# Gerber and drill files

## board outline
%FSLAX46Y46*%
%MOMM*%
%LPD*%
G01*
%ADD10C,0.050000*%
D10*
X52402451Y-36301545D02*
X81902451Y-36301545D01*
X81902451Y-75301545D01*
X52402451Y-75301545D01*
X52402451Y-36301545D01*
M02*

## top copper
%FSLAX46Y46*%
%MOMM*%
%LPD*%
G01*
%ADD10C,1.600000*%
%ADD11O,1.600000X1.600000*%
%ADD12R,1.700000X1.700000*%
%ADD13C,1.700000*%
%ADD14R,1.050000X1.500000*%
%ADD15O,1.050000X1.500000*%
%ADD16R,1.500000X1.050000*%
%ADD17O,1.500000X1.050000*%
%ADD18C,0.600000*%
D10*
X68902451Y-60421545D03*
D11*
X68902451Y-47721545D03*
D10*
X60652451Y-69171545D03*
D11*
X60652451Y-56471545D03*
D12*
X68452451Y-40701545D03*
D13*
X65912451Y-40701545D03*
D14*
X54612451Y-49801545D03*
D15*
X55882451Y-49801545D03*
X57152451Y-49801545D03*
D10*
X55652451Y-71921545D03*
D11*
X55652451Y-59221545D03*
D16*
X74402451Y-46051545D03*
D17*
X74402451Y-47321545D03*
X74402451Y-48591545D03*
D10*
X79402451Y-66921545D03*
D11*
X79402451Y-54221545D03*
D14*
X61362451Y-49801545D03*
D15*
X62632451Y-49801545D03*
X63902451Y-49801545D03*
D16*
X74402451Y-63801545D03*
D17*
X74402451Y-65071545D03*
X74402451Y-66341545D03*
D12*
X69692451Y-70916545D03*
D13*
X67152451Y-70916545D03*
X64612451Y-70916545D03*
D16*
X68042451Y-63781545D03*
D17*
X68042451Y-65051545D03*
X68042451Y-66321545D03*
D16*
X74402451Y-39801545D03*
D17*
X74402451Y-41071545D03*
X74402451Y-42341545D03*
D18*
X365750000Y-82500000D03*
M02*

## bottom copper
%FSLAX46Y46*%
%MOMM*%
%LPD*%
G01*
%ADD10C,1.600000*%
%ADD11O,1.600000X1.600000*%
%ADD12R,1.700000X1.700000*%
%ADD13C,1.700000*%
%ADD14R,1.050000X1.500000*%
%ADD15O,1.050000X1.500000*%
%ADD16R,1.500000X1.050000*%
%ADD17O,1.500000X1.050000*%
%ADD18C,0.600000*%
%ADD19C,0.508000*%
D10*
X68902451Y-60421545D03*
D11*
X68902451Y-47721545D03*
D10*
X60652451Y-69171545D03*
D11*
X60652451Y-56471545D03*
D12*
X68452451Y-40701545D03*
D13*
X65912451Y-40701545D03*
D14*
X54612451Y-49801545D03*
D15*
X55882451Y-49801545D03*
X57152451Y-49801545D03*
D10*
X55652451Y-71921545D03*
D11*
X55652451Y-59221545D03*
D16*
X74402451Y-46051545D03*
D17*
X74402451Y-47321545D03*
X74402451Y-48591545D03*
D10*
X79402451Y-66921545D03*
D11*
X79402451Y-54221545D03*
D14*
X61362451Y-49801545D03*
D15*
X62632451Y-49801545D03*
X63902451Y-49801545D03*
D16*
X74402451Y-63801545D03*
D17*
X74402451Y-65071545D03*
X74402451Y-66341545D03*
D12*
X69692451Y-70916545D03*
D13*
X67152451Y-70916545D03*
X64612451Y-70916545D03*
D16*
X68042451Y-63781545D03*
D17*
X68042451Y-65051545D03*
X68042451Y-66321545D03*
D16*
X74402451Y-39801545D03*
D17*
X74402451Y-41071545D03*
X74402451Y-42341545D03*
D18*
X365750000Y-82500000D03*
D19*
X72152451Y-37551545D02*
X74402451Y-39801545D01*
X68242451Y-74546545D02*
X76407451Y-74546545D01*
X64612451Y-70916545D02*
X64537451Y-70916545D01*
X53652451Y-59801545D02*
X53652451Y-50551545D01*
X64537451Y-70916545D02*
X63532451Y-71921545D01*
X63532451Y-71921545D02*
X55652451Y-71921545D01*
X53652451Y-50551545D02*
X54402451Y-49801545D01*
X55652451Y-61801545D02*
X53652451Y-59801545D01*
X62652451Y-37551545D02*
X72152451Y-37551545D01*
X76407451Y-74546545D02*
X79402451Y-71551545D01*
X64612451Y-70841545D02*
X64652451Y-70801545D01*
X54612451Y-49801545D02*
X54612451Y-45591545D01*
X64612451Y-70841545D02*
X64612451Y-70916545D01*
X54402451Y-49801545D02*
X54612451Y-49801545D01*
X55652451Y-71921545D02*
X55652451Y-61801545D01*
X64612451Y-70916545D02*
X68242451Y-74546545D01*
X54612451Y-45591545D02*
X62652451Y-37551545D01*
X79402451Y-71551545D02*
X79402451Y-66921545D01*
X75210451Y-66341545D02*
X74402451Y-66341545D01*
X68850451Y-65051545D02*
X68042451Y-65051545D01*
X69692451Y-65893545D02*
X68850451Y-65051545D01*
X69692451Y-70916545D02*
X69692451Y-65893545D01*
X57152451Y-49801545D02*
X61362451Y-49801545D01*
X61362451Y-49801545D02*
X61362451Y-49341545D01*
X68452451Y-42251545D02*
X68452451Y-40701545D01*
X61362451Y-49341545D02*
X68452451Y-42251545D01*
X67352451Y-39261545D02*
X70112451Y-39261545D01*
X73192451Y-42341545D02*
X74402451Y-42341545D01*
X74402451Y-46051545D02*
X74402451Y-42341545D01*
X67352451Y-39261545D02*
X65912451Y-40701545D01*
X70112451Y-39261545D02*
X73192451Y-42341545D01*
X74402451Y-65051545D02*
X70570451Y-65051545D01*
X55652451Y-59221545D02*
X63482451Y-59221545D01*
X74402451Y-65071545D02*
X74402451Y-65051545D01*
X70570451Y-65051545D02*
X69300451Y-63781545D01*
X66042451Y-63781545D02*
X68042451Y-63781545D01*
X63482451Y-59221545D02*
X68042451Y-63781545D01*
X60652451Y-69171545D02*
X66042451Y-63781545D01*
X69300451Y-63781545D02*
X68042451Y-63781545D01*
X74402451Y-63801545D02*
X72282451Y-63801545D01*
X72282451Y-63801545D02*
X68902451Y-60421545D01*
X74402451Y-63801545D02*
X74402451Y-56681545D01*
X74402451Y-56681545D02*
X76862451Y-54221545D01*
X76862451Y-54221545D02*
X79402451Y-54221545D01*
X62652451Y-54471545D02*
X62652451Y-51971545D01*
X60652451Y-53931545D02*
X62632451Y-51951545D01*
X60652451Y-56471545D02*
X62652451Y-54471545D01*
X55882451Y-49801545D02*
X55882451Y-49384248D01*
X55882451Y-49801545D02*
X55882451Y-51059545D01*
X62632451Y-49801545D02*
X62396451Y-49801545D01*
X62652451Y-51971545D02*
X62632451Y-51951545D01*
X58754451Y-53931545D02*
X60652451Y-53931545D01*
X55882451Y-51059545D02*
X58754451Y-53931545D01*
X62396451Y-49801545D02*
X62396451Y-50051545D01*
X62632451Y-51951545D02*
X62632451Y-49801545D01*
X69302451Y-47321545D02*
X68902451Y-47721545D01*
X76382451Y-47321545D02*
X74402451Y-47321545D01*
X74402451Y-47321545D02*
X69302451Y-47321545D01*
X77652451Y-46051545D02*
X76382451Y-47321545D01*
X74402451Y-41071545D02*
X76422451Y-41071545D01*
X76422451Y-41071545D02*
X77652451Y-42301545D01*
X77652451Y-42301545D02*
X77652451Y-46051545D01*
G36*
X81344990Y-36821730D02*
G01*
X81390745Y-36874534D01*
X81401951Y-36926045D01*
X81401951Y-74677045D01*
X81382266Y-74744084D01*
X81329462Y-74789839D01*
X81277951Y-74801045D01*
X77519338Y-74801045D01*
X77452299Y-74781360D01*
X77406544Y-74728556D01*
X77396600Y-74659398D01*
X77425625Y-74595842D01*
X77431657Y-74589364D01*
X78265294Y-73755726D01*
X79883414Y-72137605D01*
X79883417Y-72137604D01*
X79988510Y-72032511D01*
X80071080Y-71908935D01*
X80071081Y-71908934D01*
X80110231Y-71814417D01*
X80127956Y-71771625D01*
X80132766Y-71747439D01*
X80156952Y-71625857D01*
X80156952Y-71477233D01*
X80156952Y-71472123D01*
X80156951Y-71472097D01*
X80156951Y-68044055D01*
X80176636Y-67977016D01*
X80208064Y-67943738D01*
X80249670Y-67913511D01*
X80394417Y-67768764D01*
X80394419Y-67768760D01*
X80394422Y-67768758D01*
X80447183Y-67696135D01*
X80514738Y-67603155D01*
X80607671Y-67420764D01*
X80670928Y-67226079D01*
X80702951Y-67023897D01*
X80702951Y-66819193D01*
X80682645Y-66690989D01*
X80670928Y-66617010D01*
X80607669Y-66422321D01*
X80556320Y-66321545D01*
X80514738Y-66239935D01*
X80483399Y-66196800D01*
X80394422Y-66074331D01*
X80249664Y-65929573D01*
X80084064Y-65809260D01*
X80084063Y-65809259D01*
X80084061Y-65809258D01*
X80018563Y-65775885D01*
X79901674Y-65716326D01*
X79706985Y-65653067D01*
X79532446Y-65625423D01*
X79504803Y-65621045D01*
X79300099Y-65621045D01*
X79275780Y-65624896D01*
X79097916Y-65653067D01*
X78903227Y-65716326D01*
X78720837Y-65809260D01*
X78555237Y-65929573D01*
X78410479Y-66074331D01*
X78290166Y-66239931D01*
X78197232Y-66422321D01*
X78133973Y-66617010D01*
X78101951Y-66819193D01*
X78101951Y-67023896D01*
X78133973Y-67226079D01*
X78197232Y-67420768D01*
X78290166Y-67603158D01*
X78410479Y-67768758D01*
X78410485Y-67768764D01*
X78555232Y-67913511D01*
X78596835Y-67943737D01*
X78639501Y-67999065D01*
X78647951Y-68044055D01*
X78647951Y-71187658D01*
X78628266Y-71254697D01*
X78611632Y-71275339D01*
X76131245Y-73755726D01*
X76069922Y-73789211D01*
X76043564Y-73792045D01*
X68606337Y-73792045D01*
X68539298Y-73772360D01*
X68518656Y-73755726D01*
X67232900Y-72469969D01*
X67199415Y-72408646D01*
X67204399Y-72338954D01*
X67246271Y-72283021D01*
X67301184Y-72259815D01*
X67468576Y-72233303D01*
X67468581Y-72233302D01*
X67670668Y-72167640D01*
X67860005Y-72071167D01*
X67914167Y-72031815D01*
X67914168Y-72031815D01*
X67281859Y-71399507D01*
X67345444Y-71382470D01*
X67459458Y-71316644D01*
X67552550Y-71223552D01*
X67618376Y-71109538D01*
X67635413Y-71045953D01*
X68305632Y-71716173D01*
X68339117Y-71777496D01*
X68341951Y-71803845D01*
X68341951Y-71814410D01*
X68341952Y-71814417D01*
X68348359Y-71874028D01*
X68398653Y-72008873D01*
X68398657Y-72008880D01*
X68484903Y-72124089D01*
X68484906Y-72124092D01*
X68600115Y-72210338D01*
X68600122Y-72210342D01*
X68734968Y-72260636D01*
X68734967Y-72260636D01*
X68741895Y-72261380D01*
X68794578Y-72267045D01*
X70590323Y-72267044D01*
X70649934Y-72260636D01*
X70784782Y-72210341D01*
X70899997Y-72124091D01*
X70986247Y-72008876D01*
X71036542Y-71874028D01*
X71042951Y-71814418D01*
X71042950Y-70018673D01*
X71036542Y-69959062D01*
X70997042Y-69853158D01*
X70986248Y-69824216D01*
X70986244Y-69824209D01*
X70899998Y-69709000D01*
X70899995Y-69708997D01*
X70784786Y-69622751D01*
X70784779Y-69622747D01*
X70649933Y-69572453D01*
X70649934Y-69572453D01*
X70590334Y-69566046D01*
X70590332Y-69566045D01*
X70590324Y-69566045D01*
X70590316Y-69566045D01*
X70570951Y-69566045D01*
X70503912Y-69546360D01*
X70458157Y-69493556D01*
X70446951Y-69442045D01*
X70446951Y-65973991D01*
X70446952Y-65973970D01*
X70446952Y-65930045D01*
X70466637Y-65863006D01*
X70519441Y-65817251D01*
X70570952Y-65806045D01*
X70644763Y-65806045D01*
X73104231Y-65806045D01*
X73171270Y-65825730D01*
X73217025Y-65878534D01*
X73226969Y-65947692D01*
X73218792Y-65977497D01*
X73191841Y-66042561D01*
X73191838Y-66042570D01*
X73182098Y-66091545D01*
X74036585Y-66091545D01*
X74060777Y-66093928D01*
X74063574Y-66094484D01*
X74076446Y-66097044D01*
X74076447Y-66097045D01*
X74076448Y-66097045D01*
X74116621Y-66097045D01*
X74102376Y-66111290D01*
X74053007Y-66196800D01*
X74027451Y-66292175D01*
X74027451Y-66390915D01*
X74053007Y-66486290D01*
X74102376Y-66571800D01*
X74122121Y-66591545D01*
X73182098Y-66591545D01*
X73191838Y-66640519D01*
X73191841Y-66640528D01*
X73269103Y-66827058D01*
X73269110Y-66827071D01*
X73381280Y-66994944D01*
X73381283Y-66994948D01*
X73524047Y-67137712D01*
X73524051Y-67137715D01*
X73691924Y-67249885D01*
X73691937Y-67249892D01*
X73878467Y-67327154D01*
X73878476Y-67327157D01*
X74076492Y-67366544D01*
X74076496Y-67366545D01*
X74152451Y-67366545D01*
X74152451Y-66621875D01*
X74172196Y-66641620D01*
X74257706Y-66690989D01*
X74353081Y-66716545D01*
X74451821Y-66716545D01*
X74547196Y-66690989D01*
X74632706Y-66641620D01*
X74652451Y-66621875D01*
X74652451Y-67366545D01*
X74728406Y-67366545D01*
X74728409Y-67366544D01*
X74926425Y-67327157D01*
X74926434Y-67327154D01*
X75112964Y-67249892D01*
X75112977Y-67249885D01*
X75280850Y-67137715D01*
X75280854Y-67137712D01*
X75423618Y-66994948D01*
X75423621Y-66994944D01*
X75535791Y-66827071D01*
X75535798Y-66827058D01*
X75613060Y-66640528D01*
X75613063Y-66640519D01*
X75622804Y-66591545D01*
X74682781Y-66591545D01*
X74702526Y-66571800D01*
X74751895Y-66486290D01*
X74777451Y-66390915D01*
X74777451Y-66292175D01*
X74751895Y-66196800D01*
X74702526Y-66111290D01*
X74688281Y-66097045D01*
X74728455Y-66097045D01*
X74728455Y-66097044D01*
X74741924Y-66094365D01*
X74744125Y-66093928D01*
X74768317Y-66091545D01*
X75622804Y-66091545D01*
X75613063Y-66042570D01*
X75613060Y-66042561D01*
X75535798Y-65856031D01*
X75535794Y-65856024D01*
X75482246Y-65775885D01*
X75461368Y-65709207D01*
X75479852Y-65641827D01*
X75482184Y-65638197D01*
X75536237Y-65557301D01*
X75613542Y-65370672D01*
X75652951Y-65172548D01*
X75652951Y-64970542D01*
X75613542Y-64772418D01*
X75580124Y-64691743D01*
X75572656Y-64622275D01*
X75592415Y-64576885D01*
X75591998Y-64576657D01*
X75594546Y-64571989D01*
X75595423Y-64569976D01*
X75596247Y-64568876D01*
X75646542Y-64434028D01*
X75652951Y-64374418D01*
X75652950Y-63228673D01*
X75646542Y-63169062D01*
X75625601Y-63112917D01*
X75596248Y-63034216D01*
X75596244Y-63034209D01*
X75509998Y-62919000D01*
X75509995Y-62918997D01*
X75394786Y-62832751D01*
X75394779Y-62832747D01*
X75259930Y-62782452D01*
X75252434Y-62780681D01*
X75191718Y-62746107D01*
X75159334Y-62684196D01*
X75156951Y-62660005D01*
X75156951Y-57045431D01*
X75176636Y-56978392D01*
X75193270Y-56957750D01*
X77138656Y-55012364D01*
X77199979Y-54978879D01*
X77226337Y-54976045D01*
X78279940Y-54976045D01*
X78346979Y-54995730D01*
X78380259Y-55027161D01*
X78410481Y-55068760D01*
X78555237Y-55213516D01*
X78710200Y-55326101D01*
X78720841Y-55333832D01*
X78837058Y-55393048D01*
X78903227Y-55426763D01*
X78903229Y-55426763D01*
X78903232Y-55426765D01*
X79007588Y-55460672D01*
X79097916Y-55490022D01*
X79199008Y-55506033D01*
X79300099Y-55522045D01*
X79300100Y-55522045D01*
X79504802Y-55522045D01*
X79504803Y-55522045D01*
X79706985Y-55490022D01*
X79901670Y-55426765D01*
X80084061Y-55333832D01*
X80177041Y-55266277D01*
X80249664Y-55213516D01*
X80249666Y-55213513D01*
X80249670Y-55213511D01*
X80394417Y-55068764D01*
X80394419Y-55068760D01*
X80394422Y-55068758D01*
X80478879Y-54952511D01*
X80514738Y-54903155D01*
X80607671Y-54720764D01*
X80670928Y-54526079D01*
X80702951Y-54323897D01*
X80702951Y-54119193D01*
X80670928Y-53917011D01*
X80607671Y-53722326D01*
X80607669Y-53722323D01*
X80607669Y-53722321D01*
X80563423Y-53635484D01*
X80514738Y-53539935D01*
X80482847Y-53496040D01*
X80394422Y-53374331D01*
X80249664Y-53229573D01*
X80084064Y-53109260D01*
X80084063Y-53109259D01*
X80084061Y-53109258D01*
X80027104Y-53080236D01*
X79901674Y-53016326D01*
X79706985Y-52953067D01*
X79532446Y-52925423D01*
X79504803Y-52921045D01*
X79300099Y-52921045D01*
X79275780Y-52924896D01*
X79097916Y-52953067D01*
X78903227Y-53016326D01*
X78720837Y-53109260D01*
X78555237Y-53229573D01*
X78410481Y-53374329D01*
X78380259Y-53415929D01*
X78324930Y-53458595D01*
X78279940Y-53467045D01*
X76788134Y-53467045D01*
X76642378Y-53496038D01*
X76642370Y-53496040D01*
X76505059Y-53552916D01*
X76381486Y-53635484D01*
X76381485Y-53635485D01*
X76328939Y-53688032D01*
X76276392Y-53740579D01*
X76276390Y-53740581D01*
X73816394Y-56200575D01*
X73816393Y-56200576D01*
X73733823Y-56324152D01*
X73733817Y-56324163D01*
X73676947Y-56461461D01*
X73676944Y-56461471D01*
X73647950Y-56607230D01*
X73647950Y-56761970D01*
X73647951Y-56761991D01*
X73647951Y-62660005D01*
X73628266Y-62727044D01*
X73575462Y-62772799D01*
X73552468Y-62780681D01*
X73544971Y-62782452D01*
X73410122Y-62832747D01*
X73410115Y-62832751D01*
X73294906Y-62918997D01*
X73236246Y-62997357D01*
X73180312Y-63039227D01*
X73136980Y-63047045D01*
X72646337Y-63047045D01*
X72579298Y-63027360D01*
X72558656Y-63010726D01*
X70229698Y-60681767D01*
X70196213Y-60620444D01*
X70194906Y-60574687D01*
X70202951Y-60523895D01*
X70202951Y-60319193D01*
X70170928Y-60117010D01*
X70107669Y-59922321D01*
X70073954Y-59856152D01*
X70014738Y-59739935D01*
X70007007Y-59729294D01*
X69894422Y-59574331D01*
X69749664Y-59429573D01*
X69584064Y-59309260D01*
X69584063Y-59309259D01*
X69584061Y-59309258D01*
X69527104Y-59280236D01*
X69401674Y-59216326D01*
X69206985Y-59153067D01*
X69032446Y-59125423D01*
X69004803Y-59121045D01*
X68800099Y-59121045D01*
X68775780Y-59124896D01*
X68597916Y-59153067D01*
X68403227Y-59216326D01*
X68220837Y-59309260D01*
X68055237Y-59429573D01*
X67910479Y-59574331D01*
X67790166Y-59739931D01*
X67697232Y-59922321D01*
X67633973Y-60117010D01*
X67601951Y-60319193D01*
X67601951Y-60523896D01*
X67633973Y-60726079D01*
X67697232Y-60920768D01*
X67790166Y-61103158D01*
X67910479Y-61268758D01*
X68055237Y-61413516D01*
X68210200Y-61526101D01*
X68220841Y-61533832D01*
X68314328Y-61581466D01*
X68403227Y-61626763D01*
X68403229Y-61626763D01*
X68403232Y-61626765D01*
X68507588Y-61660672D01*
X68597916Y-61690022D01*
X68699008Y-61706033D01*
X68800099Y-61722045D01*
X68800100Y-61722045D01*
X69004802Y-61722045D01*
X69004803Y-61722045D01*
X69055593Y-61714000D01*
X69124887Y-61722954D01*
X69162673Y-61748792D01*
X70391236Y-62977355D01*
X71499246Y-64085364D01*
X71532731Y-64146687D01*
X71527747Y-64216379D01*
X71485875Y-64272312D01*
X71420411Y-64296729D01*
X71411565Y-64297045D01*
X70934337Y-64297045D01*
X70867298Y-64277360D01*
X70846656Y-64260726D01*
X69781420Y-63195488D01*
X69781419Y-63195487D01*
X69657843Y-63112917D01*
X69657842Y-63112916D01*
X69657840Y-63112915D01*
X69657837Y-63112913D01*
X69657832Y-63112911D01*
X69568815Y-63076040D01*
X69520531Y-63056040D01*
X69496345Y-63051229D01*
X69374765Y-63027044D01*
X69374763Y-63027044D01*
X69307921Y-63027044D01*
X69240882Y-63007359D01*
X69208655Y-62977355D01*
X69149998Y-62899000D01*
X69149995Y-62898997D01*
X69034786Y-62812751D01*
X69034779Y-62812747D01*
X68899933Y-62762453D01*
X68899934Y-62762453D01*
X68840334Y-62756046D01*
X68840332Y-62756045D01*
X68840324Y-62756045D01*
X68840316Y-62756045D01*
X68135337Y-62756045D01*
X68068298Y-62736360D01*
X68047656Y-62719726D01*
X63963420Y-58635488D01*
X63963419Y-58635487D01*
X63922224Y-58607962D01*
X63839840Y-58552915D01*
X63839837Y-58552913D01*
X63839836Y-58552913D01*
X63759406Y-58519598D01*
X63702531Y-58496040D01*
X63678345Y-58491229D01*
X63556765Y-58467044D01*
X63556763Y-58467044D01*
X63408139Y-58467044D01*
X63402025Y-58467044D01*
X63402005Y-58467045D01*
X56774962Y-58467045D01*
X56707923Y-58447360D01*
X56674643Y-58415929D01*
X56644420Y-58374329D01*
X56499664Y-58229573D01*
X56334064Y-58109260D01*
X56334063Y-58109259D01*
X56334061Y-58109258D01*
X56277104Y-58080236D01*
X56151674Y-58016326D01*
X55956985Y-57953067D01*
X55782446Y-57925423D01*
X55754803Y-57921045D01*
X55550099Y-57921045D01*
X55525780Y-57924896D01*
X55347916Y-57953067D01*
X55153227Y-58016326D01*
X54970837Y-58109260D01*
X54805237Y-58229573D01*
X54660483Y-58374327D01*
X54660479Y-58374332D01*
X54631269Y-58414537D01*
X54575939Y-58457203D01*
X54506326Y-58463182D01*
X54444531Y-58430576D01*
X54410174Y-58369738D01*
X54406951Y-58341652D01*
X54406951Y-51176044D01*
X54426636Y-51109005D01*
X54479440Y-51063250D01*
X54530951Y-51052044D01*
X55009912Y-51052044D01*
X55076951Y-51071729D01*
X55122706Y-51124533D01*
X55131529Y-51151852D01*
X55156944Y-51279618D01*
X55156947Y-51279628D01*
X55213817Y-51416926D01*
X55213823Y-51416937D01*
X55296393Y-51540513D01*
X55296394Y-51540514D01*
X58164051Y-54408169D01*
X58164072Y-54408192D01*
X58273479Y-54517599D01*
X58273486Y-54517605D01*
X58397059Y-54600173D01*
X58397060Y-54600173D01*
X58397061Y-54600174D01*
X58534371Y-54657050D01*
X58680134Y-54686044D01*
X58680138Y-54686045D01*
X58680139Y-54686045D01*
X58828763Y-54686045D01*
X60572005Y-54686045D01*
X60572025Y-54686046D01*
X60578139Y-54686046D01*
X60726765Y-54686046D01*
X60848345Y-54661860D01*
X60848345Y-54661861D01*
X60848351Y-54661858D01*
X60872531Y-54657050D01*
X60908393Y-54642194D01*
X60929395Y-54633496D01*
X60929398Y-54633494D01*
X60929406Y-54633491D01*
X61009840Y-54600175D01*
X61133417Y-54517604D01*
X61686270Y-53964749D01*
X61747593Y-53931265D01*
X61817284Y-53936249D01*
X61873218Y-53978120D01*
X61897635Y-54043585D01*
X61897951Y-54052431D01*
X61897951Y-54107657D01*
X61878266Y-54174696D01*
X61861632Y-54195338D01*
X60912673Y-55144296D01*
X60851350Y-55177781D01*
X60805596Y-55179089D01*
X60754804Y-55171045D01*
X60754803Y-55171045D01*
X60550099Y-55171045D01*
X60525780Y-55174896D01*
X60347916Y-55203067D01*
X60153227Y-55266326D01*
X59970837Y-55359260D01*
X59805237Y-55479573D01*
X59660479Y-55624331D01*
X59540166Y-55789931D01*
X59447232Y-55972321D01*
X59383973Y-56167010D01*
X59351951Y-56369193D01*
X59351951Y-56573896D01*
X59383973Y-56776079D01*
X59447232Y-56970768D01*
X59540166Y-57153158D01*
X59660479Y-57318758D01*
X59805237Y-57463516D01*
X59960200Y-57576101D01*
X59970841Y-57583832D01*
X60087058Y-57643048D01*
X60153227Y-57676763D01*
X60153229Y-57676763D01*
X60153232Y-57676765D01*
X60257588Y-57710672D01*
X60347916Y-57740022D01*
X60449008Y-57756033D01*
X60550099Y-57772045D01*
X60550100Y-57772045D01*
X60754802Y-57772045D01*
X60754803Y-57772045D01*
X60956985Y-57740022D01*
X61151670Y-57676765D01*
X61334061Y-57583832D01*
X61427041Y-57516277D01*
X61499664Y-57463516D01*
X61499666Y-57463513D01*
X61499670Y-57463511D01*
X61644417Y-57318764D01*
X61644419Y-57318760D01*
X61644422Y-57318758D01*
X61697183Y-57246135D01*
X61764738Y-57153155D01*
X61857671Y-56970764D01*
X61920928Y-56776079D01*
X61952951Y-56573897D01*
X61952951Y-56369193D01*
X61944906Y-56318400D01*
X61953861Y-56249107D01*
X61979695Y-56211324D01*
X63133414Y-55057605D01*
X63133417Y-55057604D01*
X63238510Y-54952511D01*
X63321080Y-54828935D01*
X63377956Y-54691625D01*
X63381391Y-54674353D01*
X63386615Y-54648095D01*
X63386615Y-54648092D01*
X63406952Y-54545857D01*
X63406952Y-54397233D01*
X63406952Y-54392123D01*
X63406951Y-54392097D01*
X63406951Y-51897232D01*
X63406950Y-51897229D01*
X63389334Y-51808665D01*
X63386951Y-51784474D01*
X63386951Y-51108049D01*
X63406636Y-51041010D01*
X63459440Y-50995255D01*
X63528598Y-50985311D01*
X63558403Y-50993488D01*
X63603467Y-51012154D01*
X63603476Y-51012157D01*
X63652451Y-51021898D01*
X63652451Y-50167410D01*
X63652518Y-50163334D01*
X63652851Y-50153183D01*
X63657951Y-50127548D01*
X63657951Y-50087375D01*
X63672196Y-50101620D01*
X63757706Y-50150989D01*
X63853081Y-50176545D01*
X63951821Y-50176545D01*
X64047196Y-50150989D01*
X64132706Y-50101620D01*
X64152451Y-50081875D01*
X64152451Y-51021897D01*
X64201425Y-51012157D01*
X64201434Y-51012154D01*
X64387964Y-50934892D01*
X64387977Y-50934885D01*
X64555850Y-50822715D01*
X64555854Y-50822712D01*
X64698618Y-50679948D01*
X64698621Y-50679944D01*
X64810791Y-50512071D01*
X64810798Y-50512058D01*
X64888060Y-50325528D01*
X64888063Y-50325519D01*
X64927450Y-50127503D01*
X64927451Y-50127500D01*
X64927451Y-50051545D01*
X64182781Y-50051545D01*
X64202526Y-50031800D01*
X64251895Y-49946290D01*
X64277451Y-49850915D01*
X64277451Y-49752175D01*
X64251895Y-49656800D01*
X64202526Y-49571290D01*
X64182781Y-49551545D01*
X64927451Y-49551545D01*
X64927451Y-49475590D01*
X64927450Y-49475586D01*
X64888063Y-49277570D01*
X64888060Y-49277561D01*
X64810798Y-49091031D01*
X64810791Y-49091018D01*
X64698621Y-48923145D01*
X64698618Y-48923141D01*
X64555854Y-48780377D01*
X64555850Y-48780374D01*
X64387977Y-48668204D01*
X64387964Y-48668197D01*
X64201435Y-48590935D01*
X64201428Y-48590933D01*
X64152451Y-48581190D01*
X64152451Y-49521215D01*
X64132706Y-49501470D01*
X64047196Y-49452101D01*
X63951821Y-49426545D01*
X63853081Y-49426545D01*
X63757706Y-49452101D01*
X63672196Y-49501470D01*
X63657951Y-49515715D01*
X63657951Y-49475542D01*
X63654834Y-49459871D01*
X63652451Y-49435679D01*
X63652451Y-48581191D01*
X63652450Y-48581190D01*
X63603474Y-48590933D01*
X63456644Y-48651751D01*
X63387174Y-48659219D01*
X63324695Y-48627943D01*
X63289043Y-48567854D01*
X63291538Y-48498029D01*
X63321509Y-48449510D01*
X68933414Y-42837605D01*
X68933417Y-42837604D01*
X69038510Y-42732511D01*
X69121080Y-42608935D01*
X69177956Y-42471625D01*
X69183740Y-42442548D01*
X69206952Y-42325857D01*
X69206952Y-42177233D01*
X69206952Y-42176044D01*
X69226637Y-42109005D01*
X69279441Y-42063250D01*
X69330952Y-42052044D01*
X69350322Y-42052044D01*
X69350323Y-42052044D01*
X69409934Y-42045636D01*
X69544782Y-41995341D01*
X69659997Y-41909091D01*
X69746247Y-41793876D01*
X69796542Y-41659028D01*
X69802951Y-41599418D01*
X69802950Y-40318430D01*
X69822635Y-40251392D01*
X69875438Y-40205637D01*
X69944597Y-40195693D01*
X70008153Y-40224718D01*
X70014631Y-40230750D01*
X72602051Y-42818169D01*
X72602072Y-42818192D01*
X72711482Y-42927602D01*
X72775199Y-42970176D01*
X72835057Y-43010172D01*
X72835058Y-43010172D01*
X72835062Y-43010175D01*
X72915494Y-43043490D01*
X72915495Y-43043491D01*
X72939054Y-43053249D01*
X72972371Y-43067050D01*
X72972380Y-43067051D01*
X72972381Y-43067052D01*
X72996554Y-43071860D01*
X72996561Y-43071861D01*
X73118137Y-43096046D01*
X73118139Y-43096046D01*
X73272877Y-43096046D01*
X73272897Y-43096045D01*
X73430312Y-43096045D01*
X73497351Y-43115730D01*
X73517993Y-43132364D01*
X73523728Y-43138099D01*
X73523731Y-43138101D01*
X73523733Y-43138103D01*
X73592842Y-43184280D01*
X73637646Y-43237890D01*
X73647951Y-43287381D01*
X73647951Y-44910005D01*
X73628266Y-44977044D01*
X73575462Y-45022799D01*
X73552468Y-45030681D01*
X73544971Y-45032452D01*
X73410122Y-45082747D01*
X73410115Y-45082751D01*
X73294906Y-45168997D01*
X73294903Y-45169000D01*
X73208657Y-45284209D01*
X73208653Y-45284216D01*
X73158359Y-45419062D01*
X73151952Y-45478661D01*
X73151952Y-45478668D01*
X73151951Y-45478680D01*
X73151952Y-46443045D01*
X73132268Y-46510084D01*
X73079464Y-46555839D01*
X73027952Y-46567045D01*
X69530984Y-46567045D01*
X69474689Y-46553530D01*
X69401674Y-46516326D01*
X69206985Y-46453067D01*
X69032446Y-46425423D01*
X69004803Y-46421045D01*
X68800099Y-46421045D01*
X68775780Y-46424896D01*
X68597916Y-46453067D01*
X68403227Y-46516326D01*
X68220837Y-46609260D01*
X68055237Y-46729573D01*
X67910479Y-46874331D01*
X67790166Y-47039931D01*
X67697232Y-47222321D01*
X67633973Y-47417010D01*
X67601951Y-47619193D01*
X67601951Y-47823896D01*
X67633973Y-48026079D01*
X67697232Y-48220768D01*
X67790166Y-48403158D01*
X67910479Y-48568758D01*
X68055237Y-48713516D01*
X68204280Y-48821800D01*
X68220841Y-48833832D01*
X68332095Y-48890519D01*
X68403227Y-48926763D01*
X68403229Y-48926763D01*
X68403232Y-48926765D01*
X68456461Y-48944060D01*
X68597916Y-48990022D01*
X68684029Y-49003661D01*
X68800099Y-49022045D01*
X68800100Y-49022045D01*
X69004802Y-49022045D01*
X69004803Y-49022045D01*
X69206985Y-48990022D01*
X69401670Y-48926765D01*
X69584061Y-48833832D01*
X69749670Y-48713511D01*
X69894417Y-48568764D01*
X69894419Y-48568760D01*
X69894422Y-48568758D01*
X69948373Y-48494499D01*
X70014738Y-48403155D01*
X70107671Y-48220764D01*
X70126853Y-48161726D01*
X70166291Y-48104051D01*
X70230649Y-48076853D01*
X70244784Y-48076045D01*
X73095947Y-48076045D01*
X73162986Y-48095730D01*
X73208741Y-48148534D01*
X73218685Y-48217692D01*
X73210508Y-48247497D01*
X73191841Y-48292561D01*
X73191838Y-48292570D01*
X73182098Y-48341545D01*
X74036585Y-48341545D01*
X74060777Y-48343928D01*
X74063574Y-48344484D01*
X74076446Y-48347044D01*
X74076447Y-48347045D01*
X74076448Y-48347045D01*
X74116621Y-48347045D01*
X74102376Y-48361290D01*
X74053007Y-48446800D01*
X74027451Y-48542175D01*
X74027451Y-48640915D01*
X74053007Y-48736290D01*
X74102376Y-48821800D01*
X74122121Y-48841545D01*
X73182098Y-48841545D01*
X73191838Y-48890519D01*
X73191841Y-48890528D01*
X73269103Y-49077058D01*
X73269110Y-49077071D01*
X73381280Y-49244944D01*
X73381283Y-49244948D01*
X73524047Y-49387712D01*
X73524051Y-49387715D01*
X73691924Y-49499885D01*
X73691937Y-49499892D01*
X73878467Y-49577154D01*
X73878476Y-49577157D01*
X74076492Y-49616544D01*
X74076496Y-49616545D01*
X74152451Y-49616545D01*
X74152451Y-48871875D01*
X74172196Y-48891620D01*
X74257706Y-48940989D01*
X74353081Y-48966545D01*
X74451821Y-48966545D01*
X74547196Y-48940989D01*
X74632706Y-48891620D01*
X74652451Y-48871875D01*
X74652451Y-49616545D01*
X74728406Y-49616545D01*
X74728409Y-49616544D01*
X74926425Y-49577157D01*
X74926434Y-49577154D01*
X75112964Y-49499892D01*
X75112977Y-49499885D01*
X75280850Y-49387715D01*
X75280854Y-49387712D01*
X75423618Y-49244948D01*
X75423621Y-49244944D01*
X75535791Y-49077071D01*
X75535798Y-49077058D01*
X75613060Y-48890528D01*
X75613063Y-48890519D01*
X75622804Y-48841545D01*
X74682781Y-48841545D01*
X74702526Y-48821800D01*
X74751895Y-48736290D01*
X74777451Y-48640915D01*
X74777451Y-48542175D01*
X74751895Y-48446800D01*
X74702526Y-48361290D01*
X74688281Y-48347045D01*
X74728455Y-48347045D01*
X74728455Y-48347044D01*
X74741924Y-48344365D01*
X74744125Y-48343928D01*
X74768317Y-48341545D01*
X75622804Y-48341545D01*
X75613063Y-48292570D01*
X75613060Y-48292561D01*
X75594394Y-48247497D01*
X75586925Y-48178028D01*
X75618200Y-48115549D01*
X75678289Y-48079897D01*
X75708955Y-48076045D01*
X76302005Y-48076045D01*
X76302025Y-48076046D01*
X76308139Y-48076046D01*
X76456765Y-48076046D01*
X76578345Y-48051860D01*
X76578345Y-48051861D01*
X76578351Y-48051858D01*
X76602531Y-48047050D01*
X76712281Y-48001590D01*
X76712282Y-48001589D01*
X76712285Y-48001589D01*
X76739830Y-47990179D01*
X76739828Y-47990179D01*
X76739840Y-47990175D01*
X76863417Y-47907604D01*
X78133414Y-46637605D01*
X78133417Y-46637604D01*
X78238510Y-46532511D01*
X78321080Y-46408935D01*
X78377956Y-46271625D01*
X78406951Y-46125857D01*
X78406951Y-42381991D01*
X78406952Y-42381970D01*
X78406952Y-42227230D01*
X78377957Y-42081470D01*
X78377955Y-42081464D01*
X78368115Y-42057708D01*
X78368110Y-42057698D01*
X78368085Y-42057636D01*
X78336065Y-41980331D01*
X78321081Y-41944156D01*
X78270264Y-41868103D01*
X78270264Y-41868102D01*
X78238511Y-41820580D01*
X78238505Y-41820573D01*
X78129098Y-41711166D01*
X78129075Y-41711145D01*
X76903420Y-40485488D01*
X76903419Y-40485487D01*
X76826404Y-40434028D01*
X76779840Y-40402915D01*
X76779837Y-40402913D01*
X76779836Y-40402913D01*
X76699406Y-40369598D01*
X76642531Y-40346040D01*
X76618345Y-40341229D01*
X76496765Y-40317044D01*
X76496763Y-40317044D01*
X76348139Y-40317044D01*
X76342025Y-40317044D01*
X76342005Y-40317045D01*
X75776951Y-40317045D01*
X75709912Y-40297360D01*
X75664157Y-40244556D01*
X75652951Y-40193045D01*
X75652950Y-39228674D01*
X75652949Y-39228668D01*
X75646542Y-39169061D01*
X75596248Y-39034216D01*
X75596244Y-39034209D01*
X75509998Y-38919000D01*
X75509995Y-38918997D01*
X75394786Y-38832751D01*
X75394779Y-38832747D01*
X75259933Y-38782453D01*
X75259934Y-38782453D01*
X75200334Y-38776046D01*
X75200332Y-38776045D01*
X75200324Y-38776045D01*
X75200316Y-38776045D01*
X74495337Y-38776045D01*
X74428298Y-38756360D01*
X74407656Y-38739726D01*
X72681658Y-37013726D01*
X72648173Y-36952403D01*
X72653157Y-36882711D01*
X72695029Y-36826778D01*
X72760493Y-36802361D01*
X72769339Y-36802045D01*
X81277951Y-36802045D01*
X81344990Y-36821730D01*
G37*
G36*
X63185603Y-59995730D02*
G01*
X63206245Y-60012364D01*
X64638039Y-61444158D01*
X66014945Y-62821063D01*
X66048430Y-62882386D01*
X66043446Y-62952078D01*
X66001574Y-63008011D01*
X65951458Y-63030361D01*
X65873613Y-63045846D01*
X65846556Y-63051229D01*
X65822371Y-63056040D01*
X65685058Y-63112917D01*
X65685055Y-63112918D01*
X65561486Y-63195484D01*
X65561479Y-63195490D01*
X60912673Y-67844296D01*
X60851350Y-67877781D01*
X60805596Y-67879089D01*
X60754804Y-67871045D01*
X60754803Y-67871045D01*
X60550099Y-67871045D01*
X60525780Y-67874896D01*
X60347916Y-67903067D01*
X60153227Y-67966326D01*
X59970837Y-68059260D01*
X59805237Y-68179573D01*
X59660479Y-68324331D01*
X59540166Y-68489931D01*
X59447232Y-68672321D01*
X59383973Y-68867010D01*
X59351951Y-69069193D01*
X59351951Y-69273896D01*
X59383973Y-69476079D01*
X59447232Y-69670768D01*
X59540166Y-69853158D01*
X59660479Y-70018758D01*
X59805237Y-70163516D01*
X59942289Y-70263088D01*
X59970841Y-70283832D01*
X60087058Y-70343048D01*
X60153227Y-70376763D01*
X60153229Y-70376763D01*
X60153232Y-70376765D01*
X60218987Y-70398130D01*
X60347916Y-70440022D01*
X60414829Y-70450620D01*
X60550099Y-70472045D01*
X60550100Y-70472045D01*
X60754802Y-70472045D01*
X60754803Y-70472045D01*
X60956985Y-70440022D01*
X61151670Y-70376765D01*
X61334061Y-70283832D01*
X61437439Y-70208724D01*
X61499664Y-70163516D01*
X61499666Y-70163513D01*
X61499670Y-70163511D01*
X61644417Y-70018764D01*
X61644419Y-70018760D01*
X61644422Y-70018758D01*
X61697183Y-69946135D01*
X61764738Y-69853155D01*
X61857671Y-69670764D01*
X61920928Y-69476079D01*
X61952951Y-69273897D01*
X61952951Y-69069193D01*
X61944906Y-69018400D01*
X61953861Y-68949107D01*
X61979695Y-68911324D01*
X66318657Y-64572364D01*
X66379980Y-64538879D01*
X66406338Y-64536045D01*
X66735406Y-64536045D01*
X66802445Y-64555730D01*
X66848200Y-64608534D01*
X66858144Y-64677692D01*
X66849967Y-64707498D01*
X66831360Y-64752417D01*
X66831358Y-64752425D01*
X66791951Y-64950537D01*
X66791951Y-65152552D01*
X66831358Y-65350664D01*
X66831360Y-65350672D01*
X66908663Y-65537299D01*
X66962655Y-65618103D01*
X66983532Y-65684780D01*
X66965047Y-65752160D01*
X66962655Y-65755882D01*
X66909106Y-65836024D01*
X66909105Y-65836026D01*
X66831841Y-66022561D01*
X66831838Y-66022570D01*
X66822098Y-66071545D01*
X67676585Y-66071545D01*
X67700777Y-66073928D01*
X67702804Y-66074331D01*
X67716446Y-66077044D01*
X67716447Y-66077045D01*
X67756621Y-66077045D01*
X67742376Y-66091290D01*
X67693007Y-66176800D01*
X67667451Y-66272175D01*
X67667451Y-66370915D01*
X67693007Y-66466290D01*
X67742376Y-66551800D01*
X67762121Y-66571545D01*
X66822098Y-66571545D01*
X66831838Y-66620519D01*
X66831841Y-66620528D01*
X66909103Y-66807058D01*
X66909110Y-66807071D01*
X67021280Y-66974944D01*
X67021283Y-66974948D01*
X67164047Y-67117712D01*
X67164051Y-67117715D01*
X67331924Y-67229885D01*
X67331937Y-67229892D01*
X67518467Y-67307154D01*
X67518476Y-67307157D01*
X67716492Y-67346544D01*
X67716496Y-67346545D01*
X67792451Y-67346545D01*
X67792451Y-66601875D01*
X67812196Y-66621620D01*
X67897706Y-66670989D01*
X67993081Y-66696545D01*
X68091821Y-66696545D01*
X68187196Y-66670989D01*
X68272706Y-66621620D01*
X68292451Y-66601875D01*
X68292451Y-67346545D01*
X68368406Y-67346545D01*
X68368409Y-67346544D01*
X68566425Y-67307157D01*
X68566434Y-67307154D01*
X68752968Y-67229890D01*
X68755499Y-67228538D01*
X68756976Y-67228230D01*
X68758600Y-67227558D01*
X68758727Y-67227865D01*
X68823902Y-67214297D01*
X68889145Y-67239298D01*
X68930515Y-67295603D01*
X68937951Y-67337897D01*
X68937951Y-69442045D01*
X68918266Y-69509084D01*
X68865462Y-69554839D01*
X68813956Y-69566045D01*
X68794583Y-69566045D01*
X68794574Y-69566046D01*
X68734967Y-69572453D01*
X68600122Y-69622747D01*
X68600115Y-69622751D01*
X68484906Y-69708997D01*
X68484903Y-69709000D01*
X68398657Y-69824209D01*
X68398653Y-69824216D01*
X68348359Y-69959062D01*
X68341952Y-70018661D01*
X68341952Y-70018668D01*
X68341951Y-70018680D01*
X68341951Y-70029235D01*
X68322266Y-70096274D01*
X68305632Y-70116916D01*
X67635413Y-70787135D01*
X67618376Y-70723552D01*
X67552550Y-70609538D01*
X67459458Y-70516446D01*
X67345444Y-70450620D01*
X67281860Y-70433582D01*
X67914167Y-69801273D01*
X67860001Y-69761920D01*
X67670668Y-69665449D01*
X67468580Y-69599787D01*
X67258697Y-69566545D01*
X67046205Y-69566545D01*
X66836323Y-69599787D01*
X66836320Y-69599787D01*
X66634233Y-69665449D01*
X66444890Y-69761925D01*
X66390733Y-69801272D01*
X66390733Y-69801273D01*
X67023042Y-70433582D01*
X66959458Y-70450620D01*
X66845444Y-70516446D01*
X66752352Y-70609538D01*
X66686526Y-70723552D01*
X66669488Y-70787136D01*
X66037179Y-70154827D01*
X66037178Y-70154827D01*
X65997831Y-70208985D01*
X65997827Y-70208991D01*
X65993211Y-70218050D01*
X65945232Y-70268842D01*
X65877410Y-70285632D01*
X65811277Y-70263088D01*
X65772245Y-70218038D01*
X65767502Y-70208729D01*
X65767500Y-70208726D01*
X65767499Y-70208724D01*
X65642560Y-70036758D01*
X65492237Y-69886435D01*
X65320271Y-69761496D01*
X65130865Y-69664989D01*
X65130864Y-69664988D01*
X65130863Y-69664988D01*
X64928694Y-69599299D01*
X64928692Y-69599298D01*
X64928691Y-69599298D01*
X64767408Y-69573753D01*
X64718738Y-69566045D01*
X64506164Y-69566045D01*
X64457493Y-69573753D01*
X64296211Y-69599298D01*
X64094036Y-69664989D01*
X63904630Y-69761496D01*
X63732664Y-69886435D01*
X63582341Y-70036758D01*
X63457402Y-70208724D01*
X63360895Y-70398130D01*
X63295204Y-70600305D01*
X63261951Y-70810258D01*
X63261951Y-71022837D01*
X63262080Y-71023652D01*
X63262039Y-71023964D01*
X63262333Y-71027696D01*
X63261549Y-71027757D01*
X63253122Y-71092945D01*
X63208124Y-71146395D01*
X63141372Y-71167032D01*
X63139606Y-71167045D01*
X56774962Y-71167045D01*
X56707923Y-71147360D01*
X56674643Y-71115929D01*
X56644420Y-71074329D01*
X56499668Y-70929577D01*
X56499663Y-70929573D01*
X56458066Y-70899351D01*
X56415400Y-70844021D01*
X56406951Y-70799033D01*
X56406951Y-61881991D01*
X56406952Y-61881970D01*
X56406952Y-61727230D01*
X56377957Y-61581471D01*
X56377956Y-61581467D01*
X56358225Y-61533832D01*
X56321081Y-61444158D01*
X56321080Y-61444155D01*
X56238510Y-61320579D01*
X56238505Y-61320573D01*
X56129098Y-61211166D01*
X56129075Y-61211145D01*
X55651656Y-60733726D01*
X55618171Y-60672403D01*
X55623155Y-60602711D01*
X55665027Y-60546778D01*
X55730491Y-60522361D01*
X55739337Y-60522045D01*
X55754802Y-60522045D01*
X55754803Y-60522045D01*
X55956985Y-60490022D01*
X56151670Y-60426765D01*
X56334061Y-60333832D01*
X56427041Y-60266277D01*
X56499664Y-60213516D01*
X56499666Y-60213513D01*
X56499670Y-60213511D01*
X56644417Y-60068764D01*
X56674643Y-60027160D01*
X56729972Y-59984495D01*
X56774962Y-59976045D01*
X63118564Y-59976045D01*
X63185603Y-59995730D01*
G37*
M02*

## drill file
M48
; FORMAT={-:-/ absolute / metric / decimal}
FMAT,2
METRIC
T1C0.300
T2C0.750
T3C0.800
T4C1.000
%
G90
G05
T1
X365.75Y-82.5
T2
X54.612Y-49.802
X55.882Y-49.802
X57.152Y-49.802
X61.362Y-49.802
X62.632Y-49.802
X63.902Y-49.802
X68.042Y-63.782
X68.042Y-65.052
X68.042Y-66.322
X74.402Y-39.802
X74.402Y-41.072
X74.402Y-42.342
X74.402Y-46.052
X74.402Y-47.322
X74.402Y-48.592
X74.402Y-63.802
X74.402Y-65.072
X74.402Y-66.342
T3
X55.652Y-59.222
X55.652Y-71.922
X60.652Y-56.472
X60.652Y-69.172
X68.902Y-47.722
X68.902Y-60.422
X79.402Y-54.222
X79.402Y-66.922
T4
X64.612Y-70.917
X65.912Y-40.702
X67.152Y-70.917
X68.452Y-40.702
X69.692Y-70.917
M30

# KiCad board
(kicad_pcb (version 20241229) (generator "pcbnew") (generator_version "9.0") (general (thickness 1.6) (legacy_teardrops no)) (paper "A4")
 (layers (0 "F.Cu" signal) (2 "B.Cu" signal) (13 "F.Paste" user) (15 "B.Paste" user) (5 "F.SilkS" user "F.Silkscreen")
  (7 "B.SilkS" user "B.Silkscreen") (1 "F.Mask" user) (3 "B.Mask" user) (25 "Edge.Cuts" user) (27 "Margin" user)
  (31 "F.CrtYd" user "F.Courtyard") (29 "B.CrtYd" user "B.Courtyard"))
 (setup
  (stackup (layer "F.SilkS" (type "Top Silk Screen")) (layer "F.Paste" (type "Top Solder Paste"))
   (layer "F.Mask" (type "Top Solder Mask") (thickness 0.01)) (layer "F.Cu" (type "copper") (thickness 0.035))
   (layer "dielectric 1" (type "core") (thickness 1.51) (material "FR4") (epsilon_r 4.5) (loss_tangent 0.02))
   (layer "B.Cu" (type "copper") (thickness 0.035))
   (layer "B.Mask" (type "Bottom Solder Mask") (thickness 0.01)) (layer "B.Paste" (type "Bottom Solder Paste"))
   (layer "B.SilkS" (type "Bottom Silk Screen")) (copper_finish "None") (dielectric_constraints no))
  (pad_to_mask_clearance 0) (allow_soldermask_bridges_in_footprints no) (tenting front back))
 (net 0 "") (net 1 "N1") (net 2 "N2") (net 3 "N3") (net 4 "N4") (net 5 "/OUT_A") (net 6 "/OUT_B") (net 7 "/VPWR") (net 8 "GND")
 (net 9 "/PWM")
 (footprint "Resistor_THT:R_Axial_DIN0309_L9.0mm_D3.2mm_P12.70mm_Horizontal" (layer "F.Cu") (at 68.902451 60.421545 90)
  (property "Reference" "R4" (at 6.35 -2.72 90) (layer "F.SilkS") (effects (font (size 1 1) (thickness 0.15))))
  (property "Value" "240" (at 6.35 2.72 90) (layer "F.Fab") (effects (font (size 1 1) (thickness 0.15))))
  (pad "1" thru_hole circle (at 0 0 90) (size 1.6 1.6) (drill 0.8) (layers "*.Cu" "*.Mask") (remove_unused_layers no) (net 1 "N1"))
  (pad "2" thru_hole oval (at 12.7 0 90) (size 1.6 1.6) (drill 0.8) (layers "*.Cu" "*.Mask") (remove_unused_layers no) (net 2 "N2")))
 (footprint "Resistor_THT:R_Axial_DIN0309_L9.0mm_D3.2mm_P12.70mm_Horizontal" (layer "F.Cu") (at 60.652451 69.171545 90)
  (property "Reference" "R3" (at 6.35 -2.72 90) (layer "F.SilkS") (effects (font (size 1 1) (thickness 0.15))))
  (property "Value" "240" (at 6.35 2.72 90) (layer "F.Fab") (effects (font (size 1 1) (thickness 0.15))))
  (pad "1" thru_hole circle (at 0 0 90) (size 1.6 1.6) (drill 0.8) (layers "*.Cu" "*.Mask") (remove_unused_layers no) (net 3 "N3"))
  (pad "2" thru_hole oval (at 12.7 0 90) (size 1.6 1.6) (drill 0.8) (layers "*.Cu" "*.Mask") (remove_unused_layers no) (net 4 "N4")))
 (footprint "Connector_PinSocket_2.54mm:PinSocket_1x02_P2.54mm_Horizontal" (layer "F.Cu") (at 68.452451 40.701545 -90)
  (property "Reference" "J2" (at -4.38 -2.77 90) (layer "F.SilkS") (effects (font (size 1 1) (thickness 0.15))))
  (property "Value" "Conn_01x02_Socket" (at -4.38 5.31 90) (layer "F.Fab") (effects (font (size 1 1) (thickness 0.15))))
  (pad "1" thru_hole rect (at 0 0 270) (size 1.7 1.7) (drill 1) (layers "*.Cu" "*.Mask") (remove_unused_layers no) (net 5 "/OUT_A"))
  (pad "2" thru_hole circle (at 0 2.54 270) (size 1.7 1.7) (drill 1) (layers "*.Cu" "*.Mask") (remove_unused_layers no) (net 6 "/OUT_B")))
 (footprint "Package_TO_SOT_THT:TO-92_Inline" (layer "F.Cu") (at 54.612451 49.801545)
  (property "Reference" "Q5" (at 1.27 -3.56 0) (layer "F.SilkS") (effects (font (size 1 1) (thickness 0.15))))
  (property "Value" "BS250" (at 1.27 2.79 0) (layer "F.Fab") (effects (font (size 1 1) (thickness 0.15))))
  (pad "1" thru_hole rect (at 0 0) (size 1.05 1.5) (drill 0.75) (layers "*.Cu" "*.Mask") (remove_unused_layers no) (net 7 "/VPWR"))
  (pad "2" thru_hole oval (at 1.27 0) (size 1.05 1.5) (drill 0.75) (layers "*.Cu" "*.Mask") (remove_unused_layers no) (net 4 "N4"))
  (pad "3" thru_hole oval (at 2.54 0) (size 1.05 1.5) (drill 0.75) (layers "*.Cu" "*.Mask") (remove_unused_layers no) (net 5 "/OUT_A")))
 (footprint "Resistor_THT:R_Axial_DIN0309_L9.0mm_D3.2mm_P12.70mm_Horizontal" (layer "F.Cu") (at 55.652451 71.921545 90)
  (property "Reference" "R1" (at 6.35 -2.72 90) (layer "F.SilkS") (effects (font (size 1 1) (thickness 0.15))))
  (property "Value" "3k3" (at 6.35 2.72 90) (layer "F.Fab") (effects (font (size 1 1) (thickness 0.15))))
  (pad "1" thru_hole circle (at 0 0 90) (size 1.6 1.6) (drill 0.8) (layers "*.Cu" "*.Mask") (remove_unused_layers no) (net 7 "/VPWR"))
  (pad "2" thru_hole oval (at 12.7 0 90) (size 1.6 1.6) (drill 0.8) (layers "*.Cu" "*.Mask") (remove_unused_layers no) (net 3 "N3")))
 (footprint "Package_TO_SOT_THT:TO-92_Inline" (layer "F.Cu") (at 74.402451 46.051545 -90)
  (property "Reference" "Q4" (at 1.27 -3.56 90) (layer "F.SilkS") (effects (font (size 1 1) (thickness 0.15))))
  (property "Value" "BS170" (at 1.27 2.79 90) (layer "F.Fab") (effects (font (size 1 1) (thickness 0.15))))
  (pad "1" thru_hole rect (at 0 0 270) (size 1.05 1.5) (drill 0.75) (layers "*.Cu" "*.Mask") (remove_unused_layers no) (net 6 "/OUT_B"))
  (pad "2" thru_hole oval (at 1.27 0 270) (size 1.05 1.5) (drill 0.75) (layers "*.Cu" "*.Mask") (remove_unused_layers no) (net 2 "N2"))
  (pad "3" thru_hole oval (at 2.54 0 270) (size 1.05 1.5) (drill 0.75) (layers "*.Cu" "*.Mask") (remove_unused_layers no) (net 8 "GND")))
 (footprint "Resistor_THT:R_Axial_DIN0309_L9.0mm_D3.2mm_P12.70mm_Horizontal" (layer "F.Cu") (at 79.402451 66.921545 90)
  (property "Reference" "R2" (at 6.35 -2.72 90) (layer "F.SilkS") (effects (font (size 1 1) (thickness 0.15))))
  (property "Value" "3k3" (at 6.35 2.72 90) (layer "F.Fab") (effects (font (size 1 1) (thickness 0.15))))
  (pad "1" thru_hole circle (at 0 0 90) (size 1.6 1.6) (drill 0.8) (layers "*.Cu" "*.Mask") (remove_unused_layers no) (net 7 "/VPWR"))
  (pad "2" thru_hole oval (at 12.7 0 90) (size 1.6 1.6) (drill 0.8) (layers "*.Cu" "*.Mask") (remove_unused_layers no) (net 1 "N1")))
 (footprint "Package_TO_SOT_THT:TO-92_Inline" (layer "F.Cu") (at 61.362451 49.801545)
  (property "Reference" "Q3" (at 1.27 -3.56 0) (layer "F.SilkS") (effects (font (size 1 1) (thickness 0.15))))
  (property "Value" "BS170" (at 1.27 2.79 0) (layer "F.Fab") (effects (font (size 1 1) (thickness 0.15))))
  (pad "1" thru_hole rect (at 0 0) (size 1.05 1.5) (drill 0.75) (layers "*.Cu" "*.Mask") (remove_unused_layers no) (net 5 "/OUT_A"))
  (pad "2" thru_hole oval (at 1.27 0) (size 1.05 1.5) (drill 0.75) (layers "*.Cu" "*.Mask") (remove_unused_layers no) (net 4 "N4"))
  (pad "3" thru_hole oval (at 2.54 0) (size 1.05 1.5) (drill 0.75) (layers "*.Cu" "*.Mask") (remove_unused_layers no) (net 8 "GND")))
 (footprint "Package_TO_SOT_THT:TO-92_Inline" (layer "F.Cu") (at 74.402451 63.801545 -90)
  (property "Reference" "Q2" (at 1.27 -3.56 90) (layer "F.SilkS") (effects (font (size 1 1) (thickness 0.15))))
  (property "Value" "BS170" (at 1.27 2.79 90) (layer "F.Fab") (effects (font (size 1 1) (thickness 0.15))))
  (pad "1" thru_hole rect (at 0 0 270) (size 1.05 1.5) (drill 0.75) (layers "*.Cu" "*.Mask") (remove_unused_layers no) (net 1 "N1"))
  (pad "2" thru_hole oval (at 1.27 0 270) (size 1.05 1.5) (drill 0.75) (layers "*.Cu" "*.Mask") (remove_unused_layers no) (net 3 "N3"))
  (pad "3" thru_hole oval (at 2.54 0 270) (size 1.05 1.5) (drill 0.75) (layers "*.Cu" "*.Mask") (remove_unused_layers no) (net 8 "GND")))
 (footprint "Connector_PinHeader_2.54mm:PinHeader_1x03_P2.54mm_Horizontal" (layer "F.Cu") (at 69.692451 70.916545 -90)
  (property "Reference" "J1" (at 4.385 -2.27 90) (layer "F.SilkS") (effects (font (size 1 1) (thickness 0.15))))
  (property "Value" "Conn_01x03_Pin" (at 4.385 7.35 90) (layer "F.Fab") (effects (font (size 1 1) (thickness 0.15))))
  (pad "1" thru_hole rect (at 0 0 270) (size 1.7 1.7) (drill 1) (layers "*.Cu" "*.Mask") (remove_unused_layers no) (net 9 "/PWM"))
  (pad "2" thru_hole circle (at 0 2.54 270) (size 1.7 1.7) (drill 1) (layers "*.Cu" "*.Mask") (remove_unused_layers no) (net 8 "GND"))
  (pad "3" thru_hole circle (at 0 5.08 270) (size 1.7 1.7) (drill 1) (layers "*.Cu" "*.Mask") (remove_unused_layers no) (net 7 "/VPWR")))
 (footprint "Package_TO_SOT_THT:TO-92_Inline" (layer "F.Cu") (at 68.042451 63.781545 -90)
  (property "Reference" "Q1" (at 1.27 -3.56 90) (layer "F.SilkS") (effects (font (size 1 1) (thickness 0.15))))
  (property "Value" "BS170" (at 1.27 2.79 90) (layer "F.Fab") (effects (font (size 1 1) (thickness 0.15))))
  (pad "1" thru_hole rect (at 0 0 270) (size 1.05 1.5) (drill 0.75) (layers "*.Cu" "*.Mask") (remove_unused_layers no) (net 3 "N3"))
  (pad "2" thru_hole oval (at 1.27 0 270) (size 1.05 1.5) (drill 0.75) (layers "*.Cu" "*.Mask") (remove_unused_layers no) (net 9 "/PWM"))
  (pad "3" thru_hole oval (at 2.54 0 270) (size 1.05 1.5) (drill 0.75) (layers "*.Cu" "*.Mask") (remove_unused_layers no) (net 8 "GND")))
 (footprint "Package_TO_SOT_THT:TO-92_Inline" (layer "F.Cu") (at 74.402451 39.801545 -90)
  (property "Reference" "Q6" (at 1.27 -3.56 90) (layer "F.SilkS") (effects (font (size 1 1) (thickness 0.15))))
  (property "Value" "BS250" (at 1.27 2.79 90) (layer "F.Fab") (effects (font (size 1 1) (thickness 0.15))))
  (pad "1" thru_hole rect (at 0 0 270) (size 1.05 1.5) (drill 0.75) (layers "*.Cu" "*.Mask") (remove_unused_layers no) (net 7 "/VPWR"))
  (pad "2" thru_hole oval (at 1.27 0 270) (size 1.05 1.5) (drill 0.75) (layers "*.Cu" "*.Mask") (remove_unused_layers no) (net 2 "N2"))
  (pad "3" thru_hole oval (at 2.54 0 270) (size 1.05 1.5) (drill 0.75) (layers "*.Cu" "*.Mask") (remove_unused_layers no) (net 6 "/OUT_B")))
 (gr_rect (start 52.402451 36.301545) (end 81.902451 75.301545) (stroke (width 0.05) (type default)) (fill no) (layer "Edge.Cuts"))
 (via (at 365.75 82.5) (size 0.6) (drill 0.3) (layers "F.Cu" "B.Cu") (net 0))
 (segment (start 72.152451 37.551545) (end 74.402451 39.801545) (width 0.508) (layer "B.Cu") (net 7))
 (segment (start 68.242451 74.546545) (end 76.407451 74.546545) (width 0.508) (layer "B.Cu") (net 7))
 (segment (start 64.612451 70.916545) (end 64.537451 70.916545) (width 0.508) (layer "B.Cu") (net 7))
 (segment (start 53.652451 59.801545) (end 53.652451 50.551545) (width 0.508) (layer "B.Cu") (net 7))
 (segment (start 64.537451 70.916545) (end 63.532451 71.921545) (width 0.508) (layer "B.Cu") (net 7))
 (segment (start 63.532451 71.921545) (end 55.652451 71.921545) (width 0.508) (layer "B.Cu") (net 7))
 (segment (start 53.652451 50.551545) (end 54.402451 49.801545) (width 0.508) (layer "B.Cu") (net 7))
 (segment (start 55.652451 61.801545) (end 53.652451 59.801545) (width 0.508) (layer "B.Cu") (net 7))
 (segment (start 62.652451 37.551545) (end 72.152451 37.551545) (width 0.508) (layer "B.Cu") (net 7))
 (segment (start 76.407451 74.546545) (end 79.402451 71.551545) (width 0.508) (layer "B.Cu") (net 7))
 (segment (start 64.612451 70.841545) (end 64.652451 70.801545) (width 0.508) (layer "B.Cu") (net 7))
 (segment (start 54.612451 49.801545) (end 54.612451 45.591545) (width 0.508) (layer "B.Cu") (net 7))
 (segment (start 64.612451 70.841545) (end 64.612451 70.916545) (width 0.508) (layer "B.Cu") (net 7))
 (segment (start 54.402451 49.801545) (end 54.612451 49.801545) (width 0.508) (layer "B.Cu") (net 7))
 (segment (start 55.652451 71.921545) (end 55.652451 61.801545) (width 0.508) (layer "B.Cu") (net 7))
 (segment (start 64.612451 70.916545) (end 68.242451 74.546545) (width 0.508) (layer "B.Cu") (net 7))
 (segment (start 54.612451 45.591545) (end 62.652451 37.551545) (width 0.508) (layer "B.Cu") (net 7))
 (segment (start 79.402451 71.551545) (end 79.402451 66.921545) (width 0.508) (layer "B.Cu") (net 7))
 (segment (start 75.210451 66.341545) (end 74.402451 66.341545) (width 0.508) (layer "B.Cu") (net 8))
 (segment (start 68.850451 65.051545) (end 68.042451 65.051545) (width 0.508) (layer "B.Cu") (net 9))
 (segment (start 69.692451 65.893545) (end 68.850451 65.051545) (width 0.508) (layer "B.Cu") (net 9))
 (segment (start 69.692451 70.916545) (end 69.692451 65.893545) (width 0.508) (layer "B.Cu") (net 9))
 (segment (start 57.152451 49.801545) (end 61.362451 49.801545) (width 0.508) (layer "B.Cu") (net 5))
 (segment (start 61.362451 49.801545) (end 61.362451 49.341545) (width 0.508) (layer "B.Cu") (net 5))
 (segment (start 68.452451 42.251545) (end 68.452451 40.701545) (width 0.508) (layer "B.Cu") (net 5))
 (segment (start 61.362451 49.341545) (end 68.452451 42.251545) (width 0.508) (layer "B.Cu") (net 5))
 (segment (start 67.352451 39.261545) (end 70.112451 39.261545) (width 0.508) (layer "B.Cu") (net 6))
 (segment (start 73.192451 42.341545) (end 74.402451 42.341545) (width 0.508) (layer "B.Cu") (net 6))
 (segment (start 74.402451 46.051545) (end 74.402451 42.341545) (width 0.508) (layer "B.Cu") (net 6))
 (segment (start 67.352451 39.261545) (end 65.912451 40.701545) (width 0.508) (layer "B.Cu") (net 6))
 (segment (start 70.112451 39.261545) (end 73.192451 42.341545) (width 0.508) (layer "B.Cu") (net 6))
 (segment (start 74.402451 65.051545) (end 70.570451 65.051545) (width 0.508) (layer "B.Cu") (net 3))
 (segment (start 55.652451 59.221545) (end 63.482451 59.221545) (width 0.508) (layer "B.Cu") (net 3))
 (segment (start 74.402451 65.071545) (end 74.402451 65.051545) (width 0.508) (layer "B.Cu") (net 3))
 (segment (start 70.570451 65.051545) (end 69.300451 63.781545) (width 0.508) (layer "B.Cu") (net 3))
 (segment (start 66.042451 63.781545) (end 68.042451 63.781545) (width 0.508) (layer "B.Cu") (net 3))
 (segment (start 63.482451 59.221545) (end 68.042451 63.781545) (width 0.508) (layer "B.Cu") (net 3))
 (segment (start 60.652451 69.171545) (end 66.042451 63.781545) (width 0.508) (layer "B.Cu") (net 3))
 (segment (start 69.300451 63.781545) (end 68.042451 63.781545) (width 0.508) (layer "B.Cu") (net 3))
 (segment (start 74.402451 63.801545) (end 72.282451 63.801545) (width 0.508) (layer "B.Cu") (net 1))
 (segment (start 72.282451 63.801545) (end 68.902451 60.421545) (width 0.508) (layer "B.Cu") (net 1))
 (segment (start 74.402451 63.801545) (end 74.402451 56.681545) (width 0.508) (layer "B.Cu") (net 1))
 (segment (start 74.402451 56.681545) (end 76.862451 54.221545) (width 0.508) (layer "B.Cu") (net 1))
 (segment (start 76.862451 54.221545) (end 79.402451 54.221545) (width 0.508) (layer "B.Cu") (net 1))
 (segment (start 62.652451 54.471545) (end 62.652451 51.971545) (width 0.508) (layer "B.Cu") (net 4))
 (segment (start 60.652451 53.931545) (end 62.632451 51.951545) (width 0.508) (layer "B.Cu") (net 4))
 (segment (start 60.652451 56.471545) (end 62.652451 54.471545) (width 0.508) (layer "B.Cu") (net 4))
 (segment (start 55.882451 49.801545) (end 55.882451 49.384248) (width 0.508) (layer "B.Cu") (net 4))
 (segment (start 55.882451 49.801545) (end 55.882451 51.059545) (width 0.508) (layer "B.Cu") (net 4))
 (segment (start 62.632451 49.801545) (end 62.396451 49.801545) (width 0.508) (layer "B.Cu") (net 4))
 (segment (start 62.652451 51.971545) (end 62.632451 51.951545) (width 0.508) (layer "B.Cu") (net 4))
 (segment (start 58.754451 53.931545) (end 60.652451 53.931545) (width 0.508) (layer "B.Cu") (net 4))
 (segment (start 55.882451 51.059545) (end 58.754451 53.931545) (width 0.508) (layer "B.Cu") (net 4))
 (segment (start 62.396451 49.801545) (end 62.396451 50.051545) (width 0.508) (layer "B.Cu") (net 4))
 (segment (start 62.632451 51.951545) (end 62.632451 49.801545) (width 0.508) (layer "B.Cu") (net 4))
 (segment (start 69.302451 47.321545) (end 68.902451 47.721545) (width 0.508) (layer "B.Cu") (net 2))
 (segment (start 76.382451 47.321545) (end 74.402451 47.321545) (width 0.508) (layer "B.Cu") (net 2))
 (segment (start 74.402451 47.321545) (end 69.302451 47.321545) (width 0.508) (layer "B.Cu") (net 2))
 (segment (start 77.652451 46.051545) (end 76.382451 47.321545) (width 0.508) (layer "B.Cu") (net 2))
 (segment (start 74.402451 41.071545) (end 76.422451 41.071545) (width 0.508) (layer "B.Cu") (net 2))
 (segment (start 76.422451 41.071545) (end 77.652451 42.301545) (width 0.508) (layer "B.Cu") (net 2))
 (segment (start 77.652451 42.301545) (end 77.652451 46.051545) (width 0.508) (layer "B.Cu") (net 2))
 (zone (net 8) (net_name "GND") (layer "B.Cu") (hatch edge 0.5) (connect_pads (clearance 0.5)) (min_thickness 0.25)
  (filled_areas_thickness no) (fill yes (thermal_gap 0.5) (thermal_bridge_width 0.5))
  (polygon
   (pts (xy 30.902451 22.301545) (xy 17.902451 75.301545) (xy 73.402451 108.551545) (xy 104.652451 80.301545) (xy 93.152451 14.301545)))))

